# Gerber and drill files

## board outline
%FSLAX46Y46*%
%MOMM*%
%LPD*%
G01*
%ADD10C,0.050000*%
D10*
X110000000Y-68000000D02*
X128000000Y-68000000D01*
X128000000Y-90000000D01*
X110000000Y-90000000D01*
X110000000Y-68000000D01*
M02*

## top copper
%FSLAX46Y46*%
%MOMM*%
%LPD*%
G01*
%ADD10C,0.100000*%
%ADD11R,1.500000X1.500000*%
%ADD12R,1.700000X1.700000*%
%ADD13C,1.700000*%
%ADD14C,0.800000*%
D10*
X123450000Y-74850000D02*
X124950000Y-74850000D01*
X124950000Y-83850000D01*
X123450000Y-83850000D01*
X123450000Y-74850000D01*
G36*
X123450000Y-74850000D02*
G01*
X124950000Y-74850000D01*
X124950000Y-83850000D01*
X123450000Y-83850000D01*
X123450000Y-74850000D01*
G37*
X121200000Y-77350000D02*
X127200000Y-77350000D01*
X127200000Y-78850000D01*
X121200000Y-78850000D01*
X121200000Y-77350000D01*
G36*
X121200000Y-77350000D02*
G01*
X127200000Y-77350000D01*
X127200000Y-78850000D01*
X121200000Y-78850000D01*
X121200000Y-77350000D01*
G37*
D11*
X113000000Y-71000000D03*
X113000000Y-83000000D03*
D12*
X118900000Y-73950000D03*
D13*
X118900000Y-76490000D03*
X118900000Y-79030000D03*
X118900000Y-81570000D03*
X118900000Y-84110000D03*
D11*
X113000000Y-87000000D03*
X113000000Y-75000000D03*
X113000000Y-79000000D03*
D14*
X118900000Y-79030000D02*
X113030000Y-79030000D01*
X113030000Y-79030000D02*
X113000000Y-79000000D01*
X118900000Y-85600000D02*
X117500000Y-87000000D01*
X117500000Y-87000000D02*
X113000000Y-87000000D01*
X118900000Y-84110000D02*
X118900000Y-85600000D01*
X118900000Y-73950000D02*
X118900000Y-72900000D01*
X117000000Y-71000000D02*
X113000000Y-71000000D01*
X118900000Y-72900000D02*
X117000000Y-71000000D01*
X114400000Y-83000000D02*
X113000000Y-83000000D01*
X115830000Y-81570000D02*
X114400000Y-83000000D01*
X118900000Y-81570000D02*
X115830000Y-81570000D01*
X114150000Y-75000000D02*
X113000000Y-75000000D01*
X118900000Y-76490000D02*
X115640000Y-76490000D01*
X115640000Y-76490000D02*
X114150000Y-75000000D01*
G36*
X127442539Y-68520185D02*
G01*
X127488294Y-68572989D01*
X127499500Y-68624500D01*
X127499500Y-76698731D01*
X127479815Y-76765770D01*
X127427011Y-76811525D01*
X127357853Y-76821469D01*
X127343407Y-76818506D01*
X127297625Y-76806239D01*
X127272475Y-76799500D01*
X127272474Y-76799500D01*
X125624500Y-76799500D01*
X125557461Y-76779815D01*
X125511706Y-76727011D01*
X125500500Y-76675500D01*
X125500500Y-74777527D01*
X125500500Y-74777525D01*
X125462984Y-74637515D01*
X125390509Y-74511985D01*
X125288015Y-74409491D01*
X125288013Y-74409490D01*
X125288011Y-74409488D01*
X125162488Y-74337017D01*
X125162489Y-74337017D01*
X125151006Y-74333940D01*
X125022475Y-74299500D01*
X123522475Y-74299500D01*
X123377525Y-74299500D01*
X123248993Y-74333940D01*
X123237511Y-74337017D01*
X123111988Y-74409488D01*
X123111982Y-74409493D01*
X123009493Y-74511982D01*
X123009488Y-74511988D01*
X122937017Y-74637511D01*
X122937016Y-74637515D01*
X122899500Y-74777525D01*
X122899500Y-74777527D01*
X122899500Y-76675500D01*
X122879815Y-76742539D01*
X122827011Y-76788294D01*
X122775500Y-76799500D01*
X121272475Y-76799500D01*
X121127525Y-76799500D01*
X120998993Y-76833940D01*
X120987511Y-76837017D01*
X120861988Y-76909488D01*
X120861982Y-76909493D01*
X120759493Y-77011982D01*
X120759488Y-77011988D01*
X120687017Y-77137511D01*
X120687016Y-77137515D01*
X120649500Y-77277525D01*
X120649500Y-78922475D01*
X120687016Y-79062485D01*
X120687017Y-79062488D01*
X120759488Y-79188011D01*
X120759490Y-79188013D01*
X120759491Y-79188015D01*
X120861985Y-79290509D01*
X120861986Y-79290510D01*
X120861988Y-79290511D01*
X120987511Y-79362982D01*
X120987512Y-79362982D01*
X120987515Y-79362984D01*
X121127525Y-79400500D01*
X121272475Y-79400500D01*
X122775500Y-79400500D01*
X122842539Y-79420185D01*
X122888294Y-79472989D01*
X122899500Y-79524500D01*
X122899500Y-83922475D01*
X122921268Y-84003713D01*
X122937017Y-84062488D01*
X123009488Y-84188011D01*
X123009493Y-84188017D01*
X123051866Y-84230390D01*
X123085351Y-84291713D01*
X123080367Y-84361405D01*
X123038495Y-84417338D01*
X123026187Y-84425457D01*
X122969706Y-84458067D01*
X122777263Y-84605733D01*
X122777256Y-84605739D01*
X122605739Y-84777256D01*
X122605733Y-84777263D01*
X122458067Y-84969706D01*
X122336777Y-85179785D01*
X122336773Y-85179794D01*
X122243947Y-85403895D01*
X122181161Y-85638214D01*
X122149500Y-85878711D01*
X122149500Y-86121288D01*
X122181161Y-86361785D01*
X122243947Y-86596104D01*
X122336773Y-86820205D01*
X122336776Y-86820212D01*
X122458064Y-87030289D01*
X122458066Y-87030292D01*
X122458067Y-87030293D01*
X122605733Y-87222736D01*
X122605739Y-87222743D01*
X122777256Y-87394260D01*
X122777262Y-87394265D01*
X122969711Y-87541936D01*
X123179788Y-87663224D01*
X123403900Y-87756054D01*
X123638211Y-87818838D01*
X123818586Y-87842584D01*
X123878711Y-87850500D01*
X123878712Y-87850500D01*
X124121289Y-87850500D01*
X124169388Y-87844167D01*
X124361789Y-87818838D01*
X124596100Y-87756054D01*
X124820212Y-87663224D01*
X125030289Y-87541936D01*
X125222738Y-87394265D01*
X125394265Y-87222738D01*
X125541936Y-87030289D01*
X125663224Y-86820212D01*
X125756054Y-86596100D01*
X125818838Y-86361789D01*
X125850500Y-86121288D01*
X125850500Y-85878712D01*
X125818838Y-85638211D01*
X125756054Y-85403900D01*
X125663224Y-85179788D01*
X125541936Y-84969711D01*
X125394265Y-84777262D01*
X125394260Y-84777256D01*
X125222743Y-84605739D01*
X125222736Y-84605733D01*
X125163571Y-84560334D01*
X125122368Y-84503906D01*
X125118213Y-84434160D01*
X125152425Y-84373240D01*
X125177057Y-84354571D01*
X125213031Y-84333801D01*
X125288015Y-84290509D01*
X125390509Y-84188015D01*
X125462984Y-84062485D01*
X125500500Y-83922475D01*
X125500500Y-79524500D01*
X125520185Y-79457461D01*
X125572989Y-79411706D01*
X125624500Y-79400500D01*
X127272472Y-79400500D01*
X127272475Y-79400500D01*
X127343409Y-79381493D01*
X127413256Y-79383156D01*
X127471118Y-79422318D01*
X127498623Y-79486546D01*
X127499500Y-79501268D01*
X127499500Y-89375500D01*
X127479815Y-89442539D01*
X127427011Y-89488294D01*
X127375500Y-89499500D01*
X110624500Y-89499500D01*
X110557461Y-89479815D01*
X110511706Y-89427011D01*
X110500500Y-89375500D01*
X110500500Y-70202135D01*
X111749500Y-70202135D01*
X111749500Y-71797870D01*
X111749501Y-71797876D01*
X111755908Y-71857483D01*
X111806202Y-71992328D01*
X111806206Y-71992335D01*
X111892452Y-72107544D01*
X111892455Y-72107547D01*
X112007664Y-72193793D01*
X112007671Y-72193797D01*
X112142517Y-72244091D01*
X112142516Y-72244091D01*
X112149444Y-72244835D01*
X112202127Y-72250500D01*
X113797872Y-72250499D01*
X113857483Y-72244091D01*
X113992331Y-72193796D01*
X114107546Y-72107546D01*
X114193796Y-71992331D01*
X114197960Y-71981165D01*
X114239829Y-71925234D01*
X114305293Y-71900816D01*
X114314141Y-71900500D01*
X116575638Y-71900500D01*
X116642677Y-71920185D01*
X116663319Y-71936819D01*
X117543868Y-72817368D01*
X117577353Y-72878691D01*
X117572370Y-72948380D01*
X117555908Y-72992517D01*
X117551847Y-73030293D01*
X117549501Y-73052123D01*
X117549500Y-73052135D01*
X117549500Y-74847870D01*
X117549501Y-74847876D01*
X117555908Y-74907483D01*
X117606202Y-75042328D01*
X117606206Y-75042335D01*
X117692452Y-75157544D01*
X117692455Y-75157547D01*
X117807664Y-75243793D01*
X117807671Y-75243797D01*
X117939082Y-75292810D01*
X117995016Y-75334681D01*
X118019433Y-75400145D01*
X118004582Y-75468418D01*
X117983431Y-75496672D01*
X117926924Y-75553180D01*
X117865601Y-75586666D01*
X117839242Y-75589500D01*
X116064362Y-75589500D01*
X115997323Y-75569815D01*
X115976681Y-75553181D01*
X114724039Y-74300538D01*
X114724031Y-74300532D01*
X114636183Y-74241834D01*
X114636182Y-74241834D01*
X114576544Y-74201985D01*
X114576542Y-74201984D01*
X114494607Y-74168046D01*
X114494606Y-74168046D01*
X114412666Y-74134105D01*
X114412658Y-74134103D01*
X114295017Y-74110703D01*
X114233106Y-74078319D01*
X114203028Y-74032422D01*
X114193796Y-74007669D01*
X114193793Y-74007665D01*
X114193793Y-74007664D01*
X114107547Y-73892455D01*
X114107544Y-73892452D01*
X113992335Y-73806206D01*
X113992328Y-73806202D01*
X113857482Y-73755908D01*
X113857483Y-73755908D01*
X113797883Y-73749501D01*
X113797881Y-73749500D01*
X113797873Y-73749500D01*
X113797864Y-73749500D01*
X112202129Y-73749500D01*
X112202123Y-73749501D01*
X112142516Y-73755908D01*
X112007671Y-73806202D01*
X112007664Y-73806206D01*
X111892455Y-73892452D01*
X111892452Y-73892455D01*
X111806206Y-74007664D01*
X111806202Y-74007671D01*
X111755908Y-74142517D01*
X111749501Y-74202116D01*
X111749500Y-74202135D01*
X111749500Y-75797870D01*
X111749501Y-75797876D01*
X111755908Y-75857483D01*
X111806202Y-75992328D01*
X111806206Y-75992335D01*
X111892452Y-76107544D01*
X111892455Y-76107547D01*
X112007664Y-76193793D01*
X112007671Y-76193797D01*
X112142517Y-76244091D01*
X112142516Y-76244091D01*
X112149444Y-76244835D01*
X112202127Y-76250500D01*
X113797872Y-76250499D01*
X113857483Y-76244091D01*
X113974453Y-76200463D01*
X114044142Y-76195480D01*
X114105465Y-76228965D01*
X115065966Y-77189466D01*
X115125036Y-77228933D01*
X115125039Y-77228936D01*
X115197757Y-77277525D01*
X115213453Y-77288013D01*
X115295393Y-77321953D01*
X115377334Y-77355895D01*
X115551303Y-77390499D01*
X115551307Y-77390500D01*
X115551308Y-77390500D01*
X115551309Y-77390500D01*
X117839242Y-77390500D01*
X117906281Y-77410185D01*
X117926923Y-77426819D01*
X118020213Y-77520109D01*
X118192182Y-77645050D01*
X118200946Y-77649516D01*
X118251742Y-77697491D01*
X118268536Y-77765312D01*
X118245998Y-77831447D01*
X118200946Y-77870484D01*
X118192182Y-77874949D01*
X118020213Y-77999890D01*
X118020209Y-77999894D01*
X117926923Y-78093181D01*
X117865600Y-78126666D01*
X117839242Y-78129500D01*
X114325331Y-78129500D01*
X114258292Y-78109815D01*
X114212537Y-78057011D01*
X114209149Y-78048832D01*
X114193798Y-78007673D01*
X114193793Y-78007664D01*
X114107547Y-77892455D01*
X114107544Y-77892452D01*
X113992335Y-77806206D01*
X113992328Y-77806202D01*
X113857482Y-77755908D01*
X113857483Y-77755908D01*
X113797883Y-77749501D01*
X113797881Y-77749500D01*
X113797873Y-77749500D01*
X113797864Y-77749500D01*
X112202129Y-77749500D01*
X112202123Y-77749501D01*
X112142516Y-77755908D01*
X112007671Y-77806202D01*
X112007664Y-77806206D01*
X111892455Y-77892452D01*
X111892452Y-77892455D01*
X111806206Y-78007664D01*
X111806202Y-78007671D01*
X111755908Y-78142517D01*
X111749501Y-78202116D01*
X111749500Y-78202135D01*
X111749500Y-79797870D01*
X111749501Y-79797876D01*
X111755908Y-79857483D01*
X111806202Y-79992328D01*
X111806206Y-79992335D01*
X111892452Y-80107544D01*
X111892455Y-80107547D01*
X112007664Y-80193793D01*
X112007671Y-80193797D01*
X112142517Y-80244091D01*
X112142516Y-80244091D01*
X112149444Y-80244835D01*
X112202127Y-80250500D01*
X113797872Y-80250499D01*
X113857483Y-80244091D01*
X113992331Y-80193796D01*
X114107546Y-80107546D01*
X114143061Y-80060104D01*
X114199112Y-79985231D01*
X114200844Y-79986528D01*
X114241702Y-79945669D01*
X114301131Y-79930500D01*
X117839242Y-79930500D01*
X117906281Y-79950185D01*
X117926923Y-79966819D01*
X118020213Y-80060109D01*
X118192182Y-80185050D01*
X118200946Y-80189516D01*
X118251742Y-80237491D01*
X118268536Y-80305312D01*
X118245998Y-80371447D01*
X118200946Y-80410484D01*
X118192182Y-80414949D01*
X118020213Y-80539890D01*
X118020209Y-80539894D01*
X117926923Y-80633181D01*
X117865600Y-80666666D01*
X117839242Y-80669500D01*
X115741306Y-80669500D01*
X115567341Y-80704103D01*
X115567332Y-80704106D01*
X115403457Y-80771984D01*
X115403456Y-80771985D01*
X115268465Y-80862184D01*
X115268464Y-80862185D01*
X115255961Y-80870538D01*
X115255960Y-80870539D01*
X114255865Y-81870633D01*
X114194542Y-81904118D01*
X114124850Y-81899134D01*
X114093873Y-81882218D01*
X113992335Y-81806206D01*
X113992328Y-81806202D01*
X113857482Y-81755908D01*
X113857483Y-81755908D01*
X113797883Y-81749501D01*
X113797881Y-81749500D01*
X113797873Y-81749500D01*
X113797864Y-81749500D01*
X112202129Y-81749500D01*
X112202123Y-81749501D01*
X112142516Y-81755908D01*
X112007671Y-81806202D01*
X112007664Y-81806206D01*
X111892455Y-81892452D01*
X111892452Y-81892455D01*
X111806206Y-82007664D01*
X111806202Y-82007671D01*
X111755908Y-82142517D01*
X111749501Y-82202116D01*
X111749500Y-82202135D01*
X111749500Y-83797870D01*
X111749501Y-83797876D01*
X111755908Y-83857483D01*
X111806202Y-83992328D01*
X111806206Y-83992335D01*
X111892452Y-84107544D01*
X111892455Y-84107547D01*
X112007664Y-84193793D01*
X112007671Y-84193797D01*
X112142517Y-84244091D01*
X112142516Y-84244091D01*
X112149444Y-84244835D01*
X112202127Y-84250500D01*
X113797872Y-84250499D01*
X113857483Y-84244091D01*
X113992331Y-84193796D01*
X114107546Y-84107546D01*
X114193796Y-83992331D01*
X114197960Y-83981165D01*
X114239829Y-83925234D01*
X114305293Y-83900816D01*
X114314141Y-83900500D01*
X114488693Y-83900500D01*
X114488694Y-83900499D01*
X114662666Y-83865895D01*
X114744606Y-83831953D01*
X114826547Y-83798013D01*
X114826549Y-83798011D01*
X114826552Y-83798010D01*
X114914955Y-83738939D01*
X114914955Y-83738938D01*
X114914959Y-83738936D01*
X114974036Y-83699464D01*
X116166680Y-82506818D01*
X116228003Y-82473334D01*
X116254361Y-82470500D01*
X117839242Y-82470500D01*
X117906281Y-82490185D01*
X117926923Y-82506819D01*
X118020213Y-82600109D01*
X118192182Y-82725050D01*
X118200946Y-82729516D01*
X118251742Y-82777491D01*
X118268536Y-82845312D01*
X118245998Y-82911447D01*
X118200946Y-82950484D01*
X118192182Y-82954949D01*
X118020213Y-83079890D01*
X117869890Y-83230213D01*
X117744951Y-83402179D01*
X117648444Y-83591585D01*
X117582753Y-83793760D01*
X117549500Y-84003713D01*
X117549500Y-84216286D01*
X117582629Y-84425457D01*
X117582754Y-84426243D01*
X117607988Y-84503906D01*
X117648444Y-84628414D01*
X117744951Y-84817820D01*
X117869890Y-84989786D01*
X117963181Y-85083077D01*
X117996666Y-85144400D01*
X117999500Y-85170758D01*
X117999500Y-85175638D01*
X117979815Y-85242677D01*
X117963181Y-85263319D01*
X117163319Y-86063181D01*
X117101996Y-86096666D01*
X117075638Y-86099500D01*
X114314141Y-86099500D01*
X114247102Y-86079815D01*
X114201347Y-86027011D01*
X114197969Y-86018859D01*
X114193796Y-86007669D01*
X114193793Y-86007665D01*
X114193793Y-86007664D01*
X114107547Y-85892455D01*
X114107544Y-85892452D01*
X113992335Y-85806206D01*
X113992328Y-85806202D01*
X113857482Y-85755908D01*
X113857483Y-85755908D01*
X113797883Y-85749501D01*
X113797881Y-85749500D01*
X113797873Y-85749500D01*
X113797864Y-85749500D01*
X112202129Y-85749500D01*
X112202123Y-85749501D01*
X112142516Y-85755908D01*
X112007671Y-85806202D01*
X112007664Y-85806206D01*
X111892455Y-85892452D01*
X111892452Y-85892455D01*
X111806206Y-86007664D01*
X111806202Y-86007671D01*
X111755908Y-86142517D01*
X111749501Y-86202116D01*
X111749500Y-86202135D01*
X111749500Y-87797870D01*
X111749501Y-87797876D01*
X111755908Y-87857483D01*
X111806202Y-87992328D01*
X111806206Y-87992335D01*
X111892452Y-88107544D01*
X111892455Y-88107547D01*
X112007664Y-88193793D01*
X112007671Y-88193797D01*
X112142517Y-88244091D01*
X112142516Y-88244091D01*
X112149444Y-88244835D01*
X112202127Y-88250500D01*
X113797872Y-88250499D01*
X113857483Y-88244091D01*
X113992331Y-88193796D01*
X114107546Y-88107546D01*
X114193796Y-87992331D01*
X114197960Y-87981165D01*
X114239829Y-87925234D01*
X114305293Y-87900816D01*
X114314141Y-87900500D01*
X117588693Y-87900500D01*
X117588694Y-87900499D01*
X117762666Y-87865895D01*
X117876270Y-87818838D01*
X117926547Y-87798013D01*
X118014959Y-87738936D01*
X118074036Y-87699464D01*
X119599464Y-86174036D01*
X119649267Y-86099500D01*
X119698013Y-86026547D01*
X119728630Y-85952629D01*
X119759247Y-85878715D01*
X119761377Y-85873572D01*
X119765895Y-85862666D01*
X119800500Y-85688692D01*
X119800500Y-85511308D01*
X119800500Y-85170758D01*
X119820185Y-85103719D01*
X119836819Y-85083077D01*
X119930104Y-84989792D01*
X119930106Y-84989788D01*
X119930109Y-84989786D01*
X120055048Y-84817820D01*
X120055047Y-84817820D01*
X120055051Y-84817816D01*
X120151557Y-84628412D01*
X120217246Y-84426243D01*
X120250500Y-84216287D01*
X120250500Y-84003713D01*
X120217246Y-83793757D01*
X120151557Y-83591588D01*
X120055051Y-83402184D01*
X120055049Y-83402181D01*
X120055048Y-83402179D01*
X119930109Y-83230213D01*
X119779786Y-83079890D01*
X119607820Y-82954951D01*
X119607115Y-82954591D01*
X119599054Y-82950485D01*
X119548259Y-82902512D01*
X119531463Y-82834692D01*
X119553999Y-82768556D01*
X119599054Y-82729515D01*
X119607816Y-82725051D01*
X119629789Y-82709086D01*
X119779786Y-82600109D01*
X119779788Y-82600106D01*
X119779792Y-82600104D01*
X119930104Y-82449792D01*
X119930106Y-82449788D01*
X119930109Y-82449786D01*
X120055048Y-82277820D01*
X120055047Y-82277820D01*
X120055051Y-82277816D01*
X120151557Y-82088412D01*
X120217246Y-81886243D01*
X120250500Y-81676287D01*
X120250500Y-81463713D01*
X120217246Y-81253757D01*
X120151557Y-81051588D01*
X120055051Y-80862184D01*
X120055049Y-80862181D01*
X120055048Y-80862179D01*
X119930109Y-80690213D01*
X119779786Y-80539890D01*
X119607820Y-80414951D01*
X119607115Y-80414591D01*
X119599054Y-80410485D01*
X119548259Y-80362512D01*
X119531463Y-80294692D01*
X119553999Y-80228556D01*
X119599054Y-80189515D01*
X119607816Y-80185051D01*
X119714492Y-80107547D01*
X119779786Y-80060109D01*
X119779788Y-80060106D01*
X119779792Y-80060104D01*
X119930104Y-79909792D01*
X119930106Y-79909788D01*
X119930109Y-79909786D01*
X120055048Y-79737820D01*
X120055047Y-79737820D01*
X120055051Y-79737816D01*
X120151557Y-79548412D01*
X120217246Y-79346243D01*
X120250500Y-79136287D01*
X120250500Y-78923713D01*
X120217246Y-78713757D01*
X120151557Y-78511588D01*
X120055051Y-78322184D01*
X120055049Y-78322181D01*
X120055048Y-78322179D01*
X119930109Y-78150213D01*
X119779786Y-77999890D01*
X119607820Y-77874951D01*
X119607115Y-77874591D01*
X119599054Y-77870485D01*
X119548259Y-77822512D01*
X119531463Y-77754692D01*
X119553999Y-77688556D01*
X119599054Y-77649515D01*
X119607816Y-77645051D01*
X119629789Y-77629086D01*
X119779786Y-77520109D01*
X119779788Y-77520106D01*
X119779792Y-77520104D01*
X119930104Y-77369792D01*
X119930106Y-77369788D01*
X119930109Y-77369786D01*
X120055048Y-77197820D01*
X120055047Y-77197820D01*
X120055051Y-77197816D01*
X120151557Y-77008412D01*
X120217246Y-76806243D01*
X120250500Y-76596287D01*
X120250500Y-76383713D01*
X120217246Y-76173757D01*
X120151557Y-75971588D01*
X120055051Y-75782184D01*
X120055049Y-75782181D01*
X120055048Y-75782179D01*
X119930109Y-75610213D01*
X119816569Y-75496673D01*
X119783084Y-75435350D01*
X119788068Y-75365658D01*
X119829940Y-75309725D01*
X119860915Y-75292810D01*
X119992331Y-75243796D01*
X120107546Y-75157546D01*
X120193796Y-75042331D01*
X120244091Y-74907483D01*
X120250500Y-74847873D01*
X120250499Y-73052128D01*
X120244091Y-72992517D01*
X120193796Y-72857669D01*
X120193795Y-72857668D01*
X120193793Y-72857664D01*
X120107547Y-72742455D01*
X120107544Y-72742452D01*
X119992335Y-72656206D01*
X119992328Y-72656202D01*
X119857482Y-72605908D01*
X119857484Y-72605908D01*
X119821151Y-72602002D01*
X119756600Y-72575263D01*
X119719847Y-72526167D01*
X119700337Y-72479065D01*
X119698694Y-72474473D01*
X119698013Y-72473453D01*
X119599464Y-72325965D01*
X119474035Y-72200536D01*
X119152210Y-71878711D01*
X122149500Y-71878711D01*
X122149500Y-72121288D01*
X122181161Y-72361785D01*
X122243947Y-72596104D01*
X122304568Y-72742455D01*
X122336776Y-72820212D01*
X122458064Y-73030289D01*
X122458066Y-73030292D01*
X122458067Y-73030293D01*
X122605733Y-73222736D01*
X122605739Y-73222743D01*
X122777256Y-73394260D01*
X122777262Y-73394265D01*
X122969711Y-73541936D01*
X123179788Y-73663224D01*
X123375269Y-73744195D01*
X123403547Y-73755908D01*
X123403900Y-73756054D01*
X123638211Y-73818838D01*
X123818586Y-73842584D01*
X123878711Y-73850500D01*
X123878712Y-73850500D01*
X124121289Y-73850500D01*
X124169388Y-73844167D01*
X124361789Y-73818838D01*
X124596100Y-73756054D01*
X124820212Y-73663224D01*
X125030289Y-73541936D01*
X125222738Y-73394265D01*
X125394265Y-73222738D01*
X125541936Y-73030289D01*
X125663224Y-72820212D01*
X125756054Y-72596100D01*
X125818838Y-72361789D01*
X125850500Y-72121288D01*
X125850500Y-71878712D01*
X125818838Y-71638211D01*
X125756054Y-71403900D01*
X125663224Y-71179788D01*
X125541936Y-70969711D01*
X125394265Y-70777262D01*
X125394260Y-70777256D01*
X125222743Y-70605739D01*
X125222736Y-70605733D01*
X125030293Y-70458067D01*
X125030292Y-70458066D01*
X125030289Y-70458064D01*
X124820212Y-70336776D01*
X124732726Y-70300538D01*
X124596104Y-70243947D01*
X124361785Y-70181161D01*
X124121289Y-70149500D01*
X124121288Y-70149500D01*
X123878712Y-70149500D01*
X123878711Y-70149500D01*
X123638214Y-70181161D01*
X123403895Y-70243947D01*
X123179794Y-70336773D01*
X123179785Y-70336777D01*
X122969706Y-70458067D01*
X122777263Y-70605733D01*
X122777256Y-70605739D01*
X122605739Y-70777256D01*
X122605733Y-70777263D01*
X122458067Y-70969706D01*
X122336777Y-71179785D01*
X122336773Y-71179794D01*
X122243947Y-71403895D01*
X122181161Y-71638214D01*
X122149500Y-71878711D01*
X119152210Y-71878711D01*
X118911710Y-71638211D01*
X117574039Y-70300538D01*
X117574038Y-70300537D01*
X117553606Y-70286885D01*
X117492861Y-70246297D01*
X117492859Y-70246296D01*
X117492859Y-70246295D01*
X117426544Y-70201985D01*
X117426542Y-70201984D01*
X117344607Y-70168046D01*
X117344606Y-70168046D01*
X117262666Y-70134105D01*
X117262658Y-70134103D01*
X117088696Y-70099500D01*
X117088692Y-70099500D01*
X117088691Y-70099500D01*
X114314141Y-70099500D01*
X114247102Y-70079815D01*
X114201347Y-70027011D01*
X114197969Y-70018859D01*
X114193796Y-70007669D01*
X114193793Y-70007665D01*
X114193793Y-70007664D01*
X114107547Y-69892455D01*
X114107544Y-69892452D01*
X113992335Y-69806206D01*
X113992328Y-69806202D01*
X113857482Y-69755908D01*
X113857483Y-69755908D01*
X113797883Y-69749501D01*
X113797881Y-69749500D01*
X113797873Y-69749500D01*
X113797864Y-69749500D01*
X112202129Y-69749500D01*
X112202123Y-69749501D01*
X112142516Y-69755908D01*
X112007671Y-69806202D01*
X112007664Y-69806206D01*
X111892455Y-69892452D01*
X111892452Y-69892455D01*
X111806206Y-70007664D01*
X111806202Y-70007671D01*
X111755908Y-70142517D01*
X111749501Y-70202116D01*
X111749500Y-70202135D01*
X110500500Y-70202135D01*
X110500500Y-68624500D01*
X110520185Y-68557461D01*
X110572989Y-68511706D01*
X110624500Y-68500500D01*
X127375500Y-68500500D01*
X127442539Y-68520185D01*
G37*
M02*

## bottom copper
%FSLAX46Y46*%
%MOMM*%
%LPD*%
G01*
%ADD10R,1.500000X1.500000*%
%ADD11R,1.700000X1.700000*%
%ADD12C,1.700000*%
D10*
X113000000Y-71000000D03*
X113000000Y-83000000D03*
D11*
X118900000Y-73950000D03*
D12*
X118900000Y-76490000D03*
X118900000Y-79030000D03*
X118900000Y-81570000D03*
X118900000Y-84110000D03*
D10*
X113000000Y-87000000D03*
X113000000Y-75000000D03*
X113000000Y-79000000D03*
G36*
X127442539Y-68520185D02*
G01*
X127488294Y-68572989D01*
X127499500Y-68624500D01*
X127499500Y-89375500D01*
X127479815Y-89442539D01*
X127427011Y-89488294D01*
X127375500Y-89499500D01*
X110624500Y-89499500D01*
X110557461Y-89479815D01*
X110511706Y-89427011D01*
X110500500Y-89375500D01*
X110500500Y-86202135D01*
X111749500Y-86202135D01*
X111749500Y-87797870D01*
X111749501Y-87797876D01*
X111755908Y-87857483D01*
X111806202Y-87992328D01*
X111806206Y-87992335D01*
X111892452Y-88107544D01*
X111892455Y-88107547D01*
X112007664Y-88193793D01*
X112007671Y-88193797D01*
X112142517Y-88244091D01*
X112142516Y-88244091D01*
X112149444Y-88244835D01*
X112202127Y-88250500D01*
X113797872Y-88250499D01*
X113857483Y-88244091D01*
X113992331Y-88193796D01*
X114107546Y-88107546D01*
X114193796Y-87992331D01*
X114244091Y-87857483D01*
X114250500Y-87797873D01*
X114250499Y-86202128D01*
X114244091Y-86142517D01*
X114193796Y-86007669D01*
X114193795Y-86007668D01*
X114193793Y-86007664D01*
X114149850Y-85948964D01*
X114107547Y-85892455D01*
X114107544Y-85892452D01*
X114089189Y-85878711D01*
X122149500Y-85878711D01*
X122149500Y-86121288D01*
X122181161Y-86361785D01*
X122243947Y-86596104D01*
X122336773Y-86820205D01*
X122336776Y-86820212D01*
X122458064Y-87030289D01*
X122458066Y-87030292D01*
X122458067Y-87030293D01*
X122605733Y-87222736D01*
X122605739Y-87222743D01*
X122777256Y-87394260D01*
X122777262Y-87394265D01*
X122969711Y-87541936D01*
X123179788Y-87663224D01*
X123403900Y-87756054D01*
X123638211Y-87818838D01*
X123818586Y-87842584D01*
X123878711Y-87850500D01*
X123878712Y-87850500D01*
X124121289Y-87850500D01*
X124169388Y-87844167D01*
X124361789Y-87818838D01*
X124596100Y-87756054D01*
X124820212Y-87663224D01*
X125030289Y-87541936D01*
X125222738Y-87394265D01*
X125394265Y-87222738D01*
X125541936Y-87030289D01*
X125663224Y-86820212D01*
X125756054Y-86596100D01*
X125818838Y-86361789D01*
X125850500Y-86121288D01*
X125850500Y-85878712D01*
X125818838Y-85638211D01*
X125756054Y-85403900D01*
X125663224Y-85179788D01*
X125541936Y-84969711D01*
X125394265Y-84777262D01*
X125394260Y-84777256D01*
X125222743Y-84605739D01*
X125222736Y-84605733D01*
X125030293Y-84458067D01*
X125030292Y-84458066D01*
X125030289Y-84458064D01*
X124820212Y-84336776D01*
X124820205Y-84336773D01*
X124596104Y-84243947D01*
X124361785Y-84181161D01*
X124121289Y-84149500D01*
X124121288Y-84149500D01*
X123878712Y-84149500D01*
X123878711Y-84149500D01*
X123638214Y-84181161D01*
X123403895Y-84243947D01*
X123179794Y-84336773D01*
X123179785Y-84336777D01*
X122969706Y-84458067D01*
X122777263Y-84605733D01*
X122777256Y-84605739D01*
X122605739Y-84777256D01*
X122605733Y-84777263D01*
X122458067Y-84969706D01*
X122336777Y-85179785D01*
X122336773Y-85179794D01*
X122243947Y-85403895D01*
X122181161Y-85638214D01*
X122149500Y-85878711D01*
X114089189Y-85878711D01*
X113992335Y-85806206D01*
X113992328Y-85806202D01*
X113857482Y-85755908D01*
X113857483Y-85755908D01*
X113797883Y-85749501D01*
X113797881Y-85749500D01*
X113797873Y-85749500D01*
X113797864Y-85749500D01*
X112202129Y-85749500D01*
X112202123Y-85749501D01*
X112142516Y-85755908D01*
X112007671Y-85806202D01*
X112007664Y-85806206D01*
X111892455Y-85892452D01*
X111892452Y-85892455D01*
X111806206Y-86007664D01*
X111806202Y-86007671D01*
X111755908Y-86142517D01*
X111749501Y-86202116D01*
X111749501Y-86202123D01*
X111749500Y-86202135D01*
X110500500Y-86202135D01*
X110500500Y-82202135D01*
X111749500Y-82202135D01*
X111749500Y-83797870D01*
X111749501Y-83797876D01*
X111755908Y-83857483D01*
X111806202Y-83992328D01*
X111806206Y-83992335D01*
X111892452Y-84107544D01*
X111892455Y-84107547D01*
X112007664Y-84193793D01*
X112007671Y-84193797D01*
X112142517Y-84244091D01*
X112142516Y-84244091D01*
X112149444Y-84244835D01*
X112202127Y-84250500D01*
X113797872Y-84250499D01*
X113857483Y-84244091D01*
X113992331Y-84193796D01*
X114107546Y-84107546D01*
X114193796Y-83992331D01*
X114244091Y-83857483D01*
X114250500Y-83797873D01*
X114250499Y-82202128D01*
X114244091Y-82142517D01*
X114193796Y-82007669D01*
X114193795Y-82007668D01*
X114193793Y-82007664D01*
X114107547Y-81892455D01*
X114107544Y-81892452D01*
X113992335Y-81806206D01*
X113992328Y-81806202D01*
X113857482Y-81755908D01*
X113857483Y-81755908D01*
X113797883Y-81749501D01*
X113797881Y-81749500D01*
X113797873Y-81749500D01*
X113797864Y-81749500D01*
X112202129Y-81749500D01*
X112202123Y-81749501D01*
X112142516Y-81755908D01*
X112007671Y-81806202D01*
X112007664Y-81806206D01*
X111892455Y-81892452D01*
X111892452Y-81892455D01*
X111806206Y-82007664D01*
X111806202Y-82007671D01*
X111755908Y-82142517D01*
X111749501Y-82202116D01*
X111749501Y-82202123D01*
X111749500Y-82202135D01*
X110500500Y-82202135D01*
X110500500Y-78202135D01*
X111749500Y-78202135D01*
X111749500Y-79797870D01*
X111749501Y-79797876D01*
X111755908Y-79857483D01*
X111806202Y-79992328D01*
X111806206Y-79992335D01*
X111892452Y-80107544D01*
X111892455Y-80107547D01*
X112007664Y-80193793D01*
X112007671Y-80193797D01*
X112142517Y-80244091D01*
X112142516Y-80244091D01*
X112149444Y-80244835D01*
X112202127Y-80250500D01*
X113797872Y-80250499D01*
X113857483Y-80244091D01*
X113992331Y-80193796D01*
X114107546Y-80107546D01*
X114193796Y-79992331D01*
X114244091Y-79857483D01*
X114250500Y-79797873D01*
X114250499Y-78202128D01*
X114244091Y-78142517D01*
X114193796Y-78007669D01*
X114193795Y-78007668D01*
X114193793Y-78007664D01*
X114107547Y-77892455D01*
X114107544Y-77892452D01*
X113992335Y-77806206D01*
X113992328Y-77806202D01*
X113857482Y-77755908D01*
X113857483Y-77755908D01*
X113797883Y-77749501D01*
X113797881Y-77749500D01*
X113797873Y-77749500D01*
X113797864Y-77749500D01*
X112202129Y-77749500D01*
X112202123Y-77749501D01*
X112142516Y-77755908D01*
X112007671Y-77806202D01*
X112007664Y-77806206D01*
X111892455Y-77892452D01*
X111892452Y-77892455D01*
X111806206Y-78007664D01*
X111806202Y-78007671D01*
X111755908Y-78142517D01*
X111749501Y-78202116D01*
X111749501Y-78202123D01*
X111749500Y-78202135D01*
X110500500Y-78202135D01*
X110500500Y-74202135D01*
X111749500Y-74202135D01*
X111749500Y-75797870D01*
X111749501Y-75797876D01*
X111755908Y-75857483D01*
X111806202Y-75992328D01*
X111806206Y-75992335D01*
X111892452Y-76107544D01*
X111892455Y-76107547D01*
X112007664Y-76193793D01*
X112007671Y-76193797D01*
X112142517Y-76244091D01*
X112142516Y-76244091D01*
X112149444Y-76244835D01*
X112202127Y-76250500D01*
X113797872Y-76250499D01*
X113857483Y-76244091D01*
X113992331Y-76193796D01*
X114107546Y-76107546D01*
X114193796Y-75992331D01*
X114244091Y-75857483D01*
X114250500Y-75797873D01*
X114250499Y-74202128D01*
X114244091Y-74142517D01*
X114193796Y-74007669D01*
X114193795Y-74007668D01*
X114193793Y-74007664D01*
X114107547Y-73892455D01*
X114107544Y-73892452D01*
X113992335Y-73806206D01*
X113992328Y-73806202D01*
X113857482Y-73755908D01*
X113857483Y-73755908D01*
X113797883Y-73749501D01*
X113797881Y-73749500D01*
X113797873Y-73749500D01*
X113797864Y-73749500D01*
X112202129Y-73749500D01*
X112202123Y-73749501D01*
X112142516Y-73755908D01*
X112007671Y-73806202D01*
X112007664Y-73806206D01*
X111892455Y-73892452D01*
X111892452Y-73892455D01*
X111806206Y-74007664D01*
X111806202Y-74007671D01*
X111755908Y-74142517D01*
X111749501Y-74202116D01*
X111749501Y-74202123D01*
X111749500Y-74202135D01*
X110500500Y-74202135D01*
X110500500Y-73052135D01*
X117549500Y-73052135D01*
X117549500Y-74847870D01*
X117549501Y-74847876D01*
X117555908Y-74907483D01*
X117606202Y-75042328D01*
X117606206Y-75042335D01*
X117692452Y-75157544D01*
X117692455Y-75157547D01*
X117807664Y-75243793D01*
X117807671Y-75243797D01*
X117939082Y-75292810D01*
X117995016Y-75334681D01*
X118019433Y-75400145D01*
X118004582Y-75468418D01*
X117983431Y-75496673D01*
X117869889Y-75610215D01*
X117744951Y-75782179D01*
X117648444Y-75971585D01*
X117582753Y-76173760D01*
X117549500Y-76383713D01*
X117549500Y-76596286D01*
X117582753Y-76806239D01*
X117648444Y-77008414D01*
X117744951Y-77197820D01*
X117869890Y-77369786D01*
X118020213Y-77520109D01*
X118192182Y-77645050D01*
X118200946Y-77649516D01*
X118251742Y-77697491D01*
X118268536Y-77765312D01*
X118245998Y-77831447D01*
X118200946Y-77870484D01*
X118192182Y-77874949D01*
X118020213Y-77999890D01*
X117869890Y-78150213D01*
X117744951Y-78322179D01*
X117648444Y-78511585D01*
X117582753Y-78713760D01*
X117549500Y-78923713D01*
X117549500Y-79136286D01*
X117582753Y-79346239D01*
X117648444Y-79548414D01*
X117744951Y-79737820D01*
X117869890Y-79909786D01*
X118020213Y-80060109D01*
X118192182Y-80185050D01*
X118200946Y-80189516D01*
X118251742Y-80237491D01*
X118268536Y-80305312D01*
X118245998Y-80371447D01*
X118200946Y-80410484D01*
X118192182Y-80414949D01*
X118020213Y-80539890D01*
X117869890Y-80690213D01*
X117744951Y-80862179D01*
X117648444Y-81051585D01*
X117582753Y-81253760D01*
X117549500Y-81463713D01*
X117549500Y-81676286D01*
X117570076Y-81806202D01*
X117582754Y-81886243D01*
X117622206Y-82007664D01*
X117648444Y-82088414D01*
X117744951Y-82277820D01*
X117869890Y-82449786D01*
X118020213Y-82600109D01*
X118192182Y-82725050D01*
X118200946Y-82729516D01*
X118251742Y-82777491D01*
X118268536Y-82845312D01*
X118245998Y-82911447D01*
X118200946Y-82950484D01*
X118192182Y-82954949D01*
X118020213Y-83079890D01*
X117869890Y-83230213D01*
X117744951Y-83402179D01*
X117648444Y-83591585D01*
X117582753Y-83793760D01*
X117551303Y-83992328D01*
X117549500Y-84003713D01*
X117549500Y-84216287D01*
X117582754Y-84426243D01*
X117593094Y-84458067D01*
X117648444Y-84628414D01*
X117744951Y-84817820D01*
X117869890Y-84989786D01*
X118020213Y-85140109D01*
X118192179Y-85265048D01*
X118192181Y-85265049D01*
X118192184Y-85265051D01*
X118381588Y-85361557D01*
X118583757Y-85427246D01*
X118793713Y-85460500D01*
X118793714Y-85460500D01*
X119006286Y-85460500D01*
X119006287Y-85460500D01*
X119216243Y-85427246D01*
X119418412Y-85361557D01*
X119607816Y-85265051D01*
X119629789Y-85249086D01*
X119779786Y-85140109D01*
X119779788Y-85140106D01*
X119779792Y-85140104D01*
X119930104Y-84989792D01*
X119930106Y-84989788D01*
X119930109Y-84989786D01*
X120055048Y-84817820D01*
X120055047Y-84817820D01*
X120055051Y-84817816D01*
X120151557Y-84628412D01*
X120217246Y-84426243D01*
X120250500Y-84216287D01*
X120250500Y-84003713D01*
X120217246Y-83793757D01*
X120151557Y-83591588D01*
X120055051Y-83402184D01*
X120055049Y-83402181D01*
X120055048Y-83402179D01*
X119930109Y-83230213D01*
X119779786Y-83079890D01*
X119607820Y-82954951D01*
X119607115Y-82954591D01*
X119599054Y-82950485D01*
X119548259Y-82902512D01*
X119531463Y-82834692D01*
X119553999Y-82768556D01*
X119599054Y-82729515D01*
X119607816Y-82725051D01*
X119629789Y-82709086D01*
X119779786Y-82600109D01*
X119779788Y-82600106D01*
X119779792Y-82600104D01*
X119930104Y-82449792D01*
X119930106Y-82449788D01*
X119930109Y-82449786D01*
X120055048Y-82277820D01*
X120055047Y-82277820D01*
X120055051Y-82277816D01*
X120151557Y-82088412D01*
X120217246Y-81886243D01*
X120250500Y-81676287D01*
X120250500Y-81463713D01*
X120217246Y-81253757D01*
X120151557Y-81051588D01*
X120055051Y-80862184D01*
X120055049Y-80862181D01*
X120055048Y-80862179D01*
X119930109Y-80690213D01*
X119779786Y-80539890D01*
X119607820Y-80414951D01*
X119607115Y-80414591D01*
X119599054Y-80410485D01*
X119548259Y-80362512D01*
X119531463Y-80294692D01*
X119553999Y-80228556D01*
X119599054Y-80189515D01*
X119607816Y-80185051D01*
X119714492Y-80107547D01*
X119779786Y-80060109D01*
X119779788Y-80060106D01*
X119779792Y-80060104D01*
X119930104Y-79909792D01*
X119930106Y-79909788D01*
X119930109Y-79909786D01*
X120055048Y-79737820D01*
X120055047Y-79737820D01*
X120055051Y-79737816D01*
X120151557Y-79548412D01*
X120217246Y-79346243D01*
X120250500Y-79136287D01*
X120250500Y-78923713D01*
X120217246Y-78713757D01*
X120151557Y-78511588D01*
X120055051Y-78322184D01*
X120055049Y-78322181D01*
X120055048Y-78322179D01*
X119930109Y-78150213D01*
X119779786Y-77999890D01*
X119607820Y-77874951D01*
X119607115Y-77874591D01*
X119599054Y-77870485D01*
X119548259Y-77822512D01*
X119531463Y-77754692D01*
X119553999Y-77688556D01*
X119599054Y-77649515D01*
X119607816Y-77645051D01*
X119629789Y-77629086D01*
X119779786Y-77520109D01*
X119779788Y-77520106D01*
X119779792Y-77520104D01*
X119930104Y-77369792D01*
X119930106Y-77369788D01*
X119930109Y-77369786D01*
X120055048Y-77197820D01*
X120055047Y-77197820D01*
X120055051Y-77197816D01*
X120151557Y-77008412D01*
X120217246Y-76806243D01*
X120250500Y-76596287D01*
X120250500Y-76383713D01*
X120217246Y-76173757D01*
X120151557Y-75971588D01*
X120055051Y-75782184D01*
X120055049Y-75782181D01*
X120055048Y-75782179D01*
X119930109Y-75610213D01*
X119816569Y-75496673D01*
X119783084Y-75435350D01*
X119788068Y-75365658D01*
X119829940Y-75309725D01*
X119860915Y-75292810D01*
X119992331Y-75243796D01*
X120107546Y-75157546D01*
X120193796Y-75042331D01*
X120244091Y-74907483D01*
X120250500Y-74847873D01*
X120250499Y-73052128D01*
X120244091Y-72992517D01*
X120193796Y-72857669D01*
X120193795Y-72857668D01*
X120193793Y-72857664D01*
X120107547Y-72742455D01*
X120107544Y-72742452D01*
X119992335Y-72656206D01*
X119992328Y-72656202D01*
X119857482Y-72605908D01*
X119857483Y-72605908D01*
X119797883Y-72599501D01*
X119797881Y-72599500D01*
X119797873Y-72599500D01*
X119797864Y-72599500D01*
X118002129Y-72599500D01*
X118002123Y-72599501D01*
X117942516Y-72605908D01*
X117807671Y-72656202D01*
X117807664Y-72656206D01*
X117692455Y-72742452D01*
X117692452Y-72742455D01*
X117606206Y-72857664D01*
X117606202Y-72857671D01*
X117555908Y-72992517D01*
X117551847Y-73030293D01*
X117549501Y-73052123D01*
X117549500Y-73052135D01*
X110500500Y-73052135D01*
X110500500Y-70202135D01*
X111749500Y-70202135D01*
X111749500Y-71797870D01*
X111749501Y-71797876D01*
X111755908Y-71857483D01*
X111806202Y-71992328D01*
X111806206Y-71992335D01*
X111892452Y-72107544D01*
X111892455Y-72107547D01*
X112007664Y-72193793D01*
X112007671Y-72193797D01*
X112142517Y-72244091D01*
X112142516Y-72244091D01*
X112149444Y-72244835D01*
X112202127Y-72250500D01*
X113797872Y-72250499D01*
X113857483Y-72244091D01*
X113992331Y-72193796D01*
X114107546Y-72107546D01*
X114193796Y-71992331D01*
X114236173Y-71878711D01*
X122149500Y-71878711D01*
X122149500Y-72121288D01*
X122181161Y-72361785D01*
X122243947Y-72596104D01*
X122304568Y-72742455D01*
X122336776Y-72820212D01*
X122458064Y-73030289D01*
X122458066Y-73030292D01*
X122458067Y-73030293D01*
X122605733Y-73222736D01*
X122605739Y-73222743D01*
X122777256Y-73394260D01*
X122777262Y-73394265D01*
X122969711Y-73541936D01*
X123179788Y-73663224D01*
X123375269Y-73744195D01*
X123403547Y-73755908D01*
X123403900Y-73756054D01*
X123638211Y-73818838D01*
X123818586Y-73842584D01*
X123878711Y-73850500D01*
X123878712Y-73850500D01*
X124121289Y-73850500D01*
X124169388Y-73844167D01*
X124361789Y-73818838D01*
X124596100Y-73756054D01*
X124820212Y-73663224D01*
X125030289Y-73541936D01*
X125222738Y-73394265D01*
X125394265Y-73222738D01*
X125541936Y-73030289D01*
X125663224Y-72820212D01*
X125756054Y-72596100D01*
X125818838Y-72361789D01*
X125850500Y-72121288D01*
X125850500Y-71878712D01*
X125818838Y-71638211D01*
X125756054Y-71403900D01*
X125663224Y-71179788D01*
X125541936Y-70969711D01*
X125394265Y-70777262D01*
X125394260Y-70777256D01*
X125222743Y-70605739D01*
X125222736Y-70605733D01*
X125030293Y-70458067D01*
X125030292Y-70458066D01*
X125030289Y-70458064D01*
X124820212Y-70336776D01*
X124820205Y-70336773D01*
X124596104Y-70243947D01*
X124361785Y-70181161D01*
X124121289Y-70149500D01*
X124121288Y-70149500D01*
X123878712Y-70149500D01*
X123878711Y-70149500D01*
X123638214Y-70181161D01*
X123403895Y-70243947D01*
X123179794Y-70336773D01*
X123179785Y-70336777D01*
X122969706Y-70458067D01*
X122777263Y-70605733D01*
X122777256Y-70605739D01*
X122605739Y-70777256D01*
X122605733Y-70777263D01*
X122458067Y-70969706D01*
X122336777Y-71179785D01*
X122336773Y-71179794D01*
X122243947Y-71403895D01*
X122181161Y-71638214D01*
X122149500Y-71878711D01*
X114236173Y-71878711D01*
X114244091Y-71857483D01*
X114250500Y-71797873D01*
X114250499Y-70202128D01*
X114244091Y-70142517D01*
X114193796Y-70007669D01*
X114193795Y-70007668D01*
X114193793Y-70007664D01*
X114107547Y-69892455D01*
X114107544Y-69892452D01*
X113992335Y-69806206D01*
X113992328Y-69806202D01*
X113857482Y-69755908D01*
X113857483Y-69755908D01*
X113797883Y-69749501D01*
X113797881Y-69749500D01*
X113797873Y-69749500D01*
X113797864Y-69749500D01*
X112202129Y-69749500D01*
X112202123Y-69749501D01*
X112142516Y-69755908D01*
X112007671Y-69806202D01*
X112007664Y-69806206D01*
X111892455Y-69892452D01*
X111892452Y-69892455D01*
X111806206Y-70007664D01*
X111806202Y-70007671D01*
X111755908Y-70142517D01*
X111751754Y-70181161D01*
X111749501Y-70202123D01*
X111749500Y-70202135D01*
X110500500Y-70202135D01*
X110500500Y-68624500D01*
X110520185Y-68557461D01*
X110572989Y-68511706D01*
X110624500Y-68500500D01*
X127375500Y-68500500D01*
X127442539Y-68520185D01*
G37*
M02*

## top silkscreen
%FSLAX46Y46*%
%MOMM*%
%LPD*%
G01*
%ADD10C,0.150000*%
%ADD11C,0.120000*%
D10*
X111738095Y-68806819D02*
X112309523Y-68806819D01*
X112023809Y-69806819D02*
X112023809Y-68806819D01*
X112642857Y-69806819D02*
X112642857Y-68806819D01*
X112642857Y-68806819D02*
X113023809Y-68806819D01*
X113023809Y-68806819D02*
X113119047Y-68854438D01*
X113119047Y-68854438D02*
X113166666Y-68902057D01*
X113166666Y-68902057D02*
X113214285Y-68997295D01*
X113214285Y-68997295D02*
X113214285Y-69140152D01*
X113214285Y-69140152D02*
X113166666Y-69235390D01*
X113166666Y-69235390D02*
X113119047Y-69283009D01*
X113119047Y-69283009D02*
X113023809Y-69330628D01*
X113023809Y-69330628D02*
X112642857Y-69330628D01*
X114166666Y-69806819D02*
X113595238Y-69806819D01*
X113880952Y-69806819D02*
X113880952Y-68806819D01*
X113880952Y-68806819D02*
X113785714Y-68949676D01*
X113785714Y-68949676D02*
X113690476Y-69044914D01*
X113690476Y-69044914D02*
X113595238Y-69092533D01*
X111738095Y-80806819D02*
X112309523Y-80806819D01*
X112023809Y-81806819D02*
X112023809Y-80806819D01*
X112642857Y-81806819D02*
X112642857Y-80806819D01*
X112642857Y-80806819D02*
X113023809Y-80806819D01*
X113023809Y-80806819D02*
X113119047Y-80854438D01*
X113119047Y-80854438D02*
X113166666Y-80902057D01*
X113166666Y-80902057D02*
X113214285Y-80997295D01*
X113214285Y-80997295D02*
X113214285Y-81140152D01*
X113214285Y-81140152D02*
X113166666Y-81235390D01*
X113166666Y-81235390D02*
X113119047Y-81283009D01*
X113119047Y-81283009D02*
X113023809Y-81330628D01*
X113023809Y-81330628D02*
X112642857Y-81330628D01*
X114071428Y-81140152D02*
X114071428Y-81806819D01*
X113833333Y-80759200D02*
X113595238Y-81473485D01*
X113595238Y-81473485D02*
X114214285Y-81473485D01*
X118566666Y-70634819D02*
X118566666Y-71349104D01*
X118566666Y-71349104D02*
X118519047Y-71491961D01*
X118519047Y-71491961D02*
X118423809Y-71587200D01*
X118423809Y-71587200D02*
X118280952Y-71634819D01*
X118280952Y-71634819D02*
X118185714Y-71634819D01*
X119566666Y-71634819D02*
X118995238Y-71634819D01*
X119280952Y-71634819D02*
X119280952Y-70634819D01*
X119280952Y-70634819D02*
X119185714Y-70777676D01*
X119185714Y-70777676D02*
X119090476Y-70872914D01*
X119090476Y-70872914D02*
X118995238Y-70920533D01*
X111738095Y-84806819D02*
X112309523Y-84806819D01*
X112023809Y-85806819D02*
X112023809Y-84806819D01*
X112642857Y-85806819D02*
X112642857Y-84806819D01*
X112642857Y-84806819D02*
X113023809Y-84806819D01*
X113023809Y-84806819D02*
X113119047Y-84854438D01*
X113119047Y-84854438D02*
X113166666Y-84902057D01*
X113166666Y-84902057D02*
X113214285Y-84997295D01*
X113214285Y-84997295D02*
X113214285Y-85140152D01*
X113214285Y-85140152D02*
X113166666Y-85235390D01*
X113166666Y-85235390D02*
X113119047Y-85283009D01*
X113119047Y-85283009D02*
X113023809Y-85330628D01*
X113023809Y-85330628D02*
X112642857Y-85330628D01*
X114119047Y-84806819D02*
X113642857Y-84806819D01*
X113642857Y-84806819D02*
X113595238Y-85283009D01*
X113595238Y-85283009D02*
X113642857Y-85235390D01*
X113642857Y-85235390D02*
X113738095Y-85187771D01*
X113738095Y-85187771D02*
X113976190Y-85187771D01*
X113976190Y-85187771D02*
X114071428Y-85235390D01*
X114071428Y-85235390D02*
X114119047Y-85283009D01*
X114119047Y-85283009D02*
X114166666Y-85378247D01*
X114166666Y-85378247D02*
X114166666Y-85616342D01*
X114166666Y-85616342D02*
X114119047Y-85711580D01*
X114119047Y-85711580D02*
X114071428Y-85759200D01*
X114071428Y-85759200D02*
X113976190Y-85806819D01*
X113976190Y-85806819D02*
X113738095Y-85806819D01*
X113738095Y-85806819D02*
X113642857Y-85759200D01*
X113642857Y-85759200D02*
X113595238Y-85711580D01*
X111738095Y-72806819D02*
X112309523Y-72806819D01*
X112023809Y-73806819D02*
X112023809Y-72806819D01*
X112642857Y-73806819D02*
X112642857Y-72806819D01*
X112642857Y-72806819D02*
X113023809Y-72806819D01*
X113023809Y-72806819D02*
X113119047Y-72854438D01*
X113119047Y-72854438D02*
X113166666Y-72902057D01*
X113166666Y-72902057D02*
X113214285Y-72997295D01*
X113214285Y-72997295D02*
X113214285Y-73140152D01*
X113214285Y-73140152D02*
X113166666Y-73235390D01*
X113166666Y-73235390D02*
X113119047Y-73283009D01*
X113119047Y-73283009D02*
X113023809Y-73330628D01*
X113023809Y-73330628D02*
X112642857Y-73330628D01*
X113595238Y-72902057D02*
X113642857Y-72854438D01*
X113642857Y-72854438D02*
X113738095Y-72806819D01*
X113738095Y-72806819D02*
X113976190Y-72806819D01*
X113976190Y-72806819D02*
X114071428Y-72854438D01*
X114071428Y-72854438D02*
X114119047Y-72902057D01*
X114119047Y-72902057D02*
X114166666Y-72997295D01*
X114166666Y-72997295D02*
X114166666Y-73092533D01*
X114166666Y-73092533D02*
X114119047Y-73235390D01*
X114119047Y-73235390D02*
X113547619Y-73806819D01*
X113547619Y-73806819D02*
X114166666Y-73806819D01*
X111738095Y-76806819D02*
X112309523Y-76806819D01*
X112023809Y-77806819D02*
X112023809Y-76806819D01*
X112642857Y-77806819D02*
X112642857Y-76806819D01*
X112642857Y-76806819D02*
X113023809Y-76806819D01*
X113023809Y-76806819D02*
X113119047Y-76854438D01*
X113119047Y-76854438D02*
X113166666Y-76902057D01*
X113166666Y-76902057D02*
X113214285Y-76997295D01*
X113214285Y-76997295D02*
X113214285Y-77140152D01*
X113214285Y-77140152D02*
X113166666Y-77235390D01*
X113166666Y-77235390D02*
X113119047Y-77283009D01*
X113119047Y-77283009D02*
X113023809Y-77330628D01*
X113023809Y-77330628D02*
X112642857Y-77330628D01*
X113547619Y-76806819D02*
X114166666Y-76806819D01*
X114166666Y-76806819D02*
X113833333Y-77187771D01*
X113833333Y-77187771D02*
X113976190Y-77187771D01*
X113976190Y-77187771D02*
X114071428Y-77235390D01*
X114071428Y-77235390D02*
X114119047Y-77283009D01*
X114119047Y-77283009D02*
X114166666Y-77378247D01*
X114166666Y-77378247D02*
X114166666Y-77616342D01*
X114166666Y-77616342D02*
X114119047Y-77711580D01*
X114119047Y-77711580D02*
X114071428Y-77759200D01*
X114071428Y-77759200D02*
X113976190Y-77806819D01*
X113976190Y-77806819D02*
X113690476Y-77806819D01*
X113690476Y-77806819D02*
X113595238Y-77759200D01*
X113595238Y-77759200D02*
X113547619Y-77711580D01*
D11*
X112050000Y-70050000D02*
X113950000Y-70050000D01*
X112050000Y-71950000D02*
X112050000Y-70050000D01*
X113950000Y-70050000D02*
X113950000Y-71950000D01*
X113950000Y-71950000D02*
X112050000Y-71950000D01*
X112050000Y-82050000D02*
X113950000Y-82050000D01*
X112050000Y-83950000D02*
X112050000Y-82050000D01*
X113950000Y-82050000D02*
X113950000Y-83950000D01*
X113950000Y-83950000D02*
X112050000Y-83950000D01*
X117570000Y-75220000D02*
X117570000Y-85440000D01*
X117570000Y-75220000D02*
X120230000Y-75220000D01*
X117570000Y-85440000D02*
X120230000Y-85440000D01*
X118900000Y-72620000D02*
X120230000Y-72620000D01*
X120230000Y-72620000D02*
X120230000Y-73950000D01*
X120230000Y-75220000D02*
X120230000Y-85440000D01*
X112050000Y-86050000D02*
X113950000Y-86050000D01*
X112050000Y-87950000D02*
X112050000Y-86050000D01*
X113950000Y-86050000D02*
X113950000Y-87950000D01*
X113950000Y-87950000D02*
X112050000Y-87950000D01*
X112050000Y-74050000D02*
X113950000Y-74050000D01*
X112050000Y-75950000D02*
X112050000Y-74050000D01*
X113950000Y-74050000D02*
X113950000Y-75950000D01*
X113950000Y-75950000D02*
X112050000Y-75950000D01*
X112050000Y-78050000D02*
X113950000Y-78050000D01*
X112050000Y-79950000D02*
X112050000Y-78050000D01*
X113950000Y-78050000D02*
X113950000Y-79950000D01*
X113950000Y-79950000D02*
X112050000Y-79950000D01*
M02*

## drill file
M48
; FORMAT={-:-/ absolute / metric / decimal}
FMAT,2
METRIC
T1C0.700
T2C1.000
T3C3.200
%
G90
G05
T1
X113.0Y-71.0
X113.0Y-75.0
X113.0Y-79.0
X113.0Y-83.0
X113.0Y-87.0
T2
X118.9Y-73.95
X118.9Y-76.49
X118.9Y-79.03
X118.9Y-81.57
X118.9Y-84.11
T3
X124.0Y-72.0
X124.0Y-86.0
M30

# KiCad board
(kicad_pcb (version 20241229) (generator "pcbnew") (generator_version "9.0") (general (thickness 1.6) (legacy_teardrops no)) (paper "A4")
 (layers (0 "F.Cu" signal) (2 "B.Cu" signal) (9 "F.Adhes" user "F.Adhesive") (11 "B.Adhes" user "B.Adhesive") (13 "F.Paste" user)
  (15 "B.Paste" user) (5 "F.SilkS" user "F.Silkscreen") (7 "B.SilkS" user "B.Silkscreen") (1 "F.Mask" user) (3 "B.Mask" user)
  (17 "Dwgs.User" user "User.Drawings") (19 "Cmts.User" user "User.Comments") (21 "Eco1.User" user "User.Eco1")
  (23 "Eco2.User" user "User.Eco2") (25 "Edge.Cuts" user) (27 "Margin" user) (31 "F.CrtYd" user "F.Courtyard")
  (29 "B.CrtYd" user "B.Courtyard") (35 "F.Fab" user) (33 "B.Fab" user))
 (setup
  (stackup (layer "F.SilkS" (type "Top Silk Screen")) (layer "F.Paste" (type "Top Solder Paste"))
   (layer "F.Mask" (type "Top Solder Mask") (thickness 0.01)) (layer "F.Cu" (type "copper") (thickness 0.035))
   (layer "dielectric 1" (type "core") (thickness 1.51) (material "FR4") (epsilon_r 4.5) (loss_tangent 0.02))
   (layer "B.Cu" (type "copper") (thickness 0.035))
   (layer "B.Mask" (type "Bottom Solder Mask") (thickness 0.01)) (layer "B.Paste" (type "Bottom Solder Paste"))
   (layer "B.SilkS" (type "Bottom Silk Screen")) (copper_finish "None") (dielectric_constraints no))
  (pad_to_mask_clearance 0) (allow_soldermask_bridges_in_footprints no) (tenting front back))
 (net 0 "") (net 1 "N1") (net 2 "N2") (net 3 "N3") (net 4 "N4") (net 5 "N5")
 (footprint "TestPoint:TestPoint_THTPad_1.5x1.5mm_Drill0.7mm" (layer "F.Cu") (at 113 71)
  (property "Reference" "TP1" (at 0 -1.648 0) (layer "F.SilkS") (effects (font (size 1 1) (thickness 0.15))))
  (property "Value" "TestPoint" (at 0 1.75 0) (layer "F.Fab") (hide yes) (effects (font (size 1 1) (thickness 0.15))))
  (fp_line (start -0.95 -0.95) (end 0.95 -0.95) (stroke (width 0.12) (type solid)) (layer "F.SilkS"))
  (fp_line (start -0.95 0.95) (end -0.95 -0.95) (stroke (width 0.12) (type solid)) (layer "F.SilkS"))
  (fp_line (start 0.95 -0.95) (end 0.95 0.95) (stroke (width 0.12) (type solid)) (layer "F.SilkS"))
  (fp_line (start 0.95 0.95) (end -0.95 0.95) (stroke (width 0.12) (type solid)) (layer "F.SilkS"))
  (pad "1" thru_hole rect (at 0 0) (size 1.5 1.5) (drill 0.7) (layers "*.Cu" "*.Mask") (remove_unused_layers no) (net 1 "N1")))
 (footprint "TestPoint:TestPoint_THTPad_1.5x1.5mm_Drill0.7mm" (layer "F.Cu") (at 113 83)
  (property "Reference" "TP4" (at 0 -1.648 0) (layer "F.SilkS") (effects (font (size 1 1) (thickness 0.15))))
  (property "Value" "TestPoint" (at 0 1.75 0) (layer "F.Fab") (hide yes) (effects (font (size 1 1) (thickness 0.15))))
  (fp_line (start -0.95 -0.95) (end 0.95 -0.95) (stroke (width 0.12) (type solid)) (layer "F.SilkS"))
  (fp_line (start -0.95 0.95) (end -0.95 -0.95) (stroke (width 0.12) (type solid)) (layer "F.SilkS"))
  (fp_line (start 0.95 -0.95) (end 0.95 0.95) (stroke (width 0.12) (type solid)) (layer "F.SilkS"))
  (fp_line (start 0.95 0.95) (end -0.95 0.95) (stroke (width 0.12) (type solid)) (layer "F.SilkS"))
  (pad "1" thru_hole rect (at 0 0) (size 1.5 1.5) (drill 0.7) (layers "*.Cu" "*.Mask") (remove_unused_layers no) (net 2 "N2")))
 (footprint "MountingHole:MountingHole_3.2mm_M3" (layer "F.Cu") (at 124 72)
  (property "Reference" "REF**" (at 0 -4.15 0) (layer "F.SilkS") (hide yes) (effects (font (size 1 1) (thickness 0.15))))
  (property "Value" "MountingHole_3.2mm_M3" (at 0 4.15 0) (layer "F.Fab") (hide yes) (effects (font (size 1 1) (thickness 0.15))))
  (pad "" np_thru_hole circle (at 0 0) (size 3.2 3.2) (drill 3.2) (layers "*.Cu" "*.Mask")))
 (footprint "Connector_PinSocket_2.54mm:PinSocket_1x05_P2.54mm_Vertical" (layer "F.Cu") (at 118.9 73.95)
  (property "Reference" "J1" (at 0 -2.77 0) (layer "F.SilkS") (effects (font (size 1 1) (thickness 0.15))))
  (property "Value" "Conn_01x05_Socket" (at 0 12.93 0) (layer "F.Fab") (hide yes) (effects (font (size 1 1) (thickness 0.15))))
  (fp_line (start -1.33 1.27) (end -1.33 11.49) (stroke (width 0.12) (type solid)) (layer "F.SilkS"))
  (fp_line (start -1.33 1.27) (end 1.33 1.27) (stroke (width 0.12) (type solid)) (layer "F.SilkS"))
  (fp_line (start -1.33 11.49) (end 1.33 11.49) (stroke (width 0.12) (type solid)) (layer "F.SilkS"))
  (fp_line (start 0 -1.33) (end 1.33 -1.33) (stroke (width 0.12) (type solid)) (layer "F.SilkS"))
  (fp_line (start 1.33 -1.33) (end 1.33 0) (stroke (width 0.12) (type solid)) (layer "F.SilkS"))
  (fp_line (start 1.33 1.27) (end 1.33 11.49) (stroke (width 0.12) (type solid)) (layer "F.SilkS"))
  (pad "1" thru_hole rect (at 0 0) (size 1.7 1.7) (drill 1) (layers "*.Cu" "*.Mask") (remove_unused_layers no) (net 1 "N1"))
  (pad "2" thru_hole circle (at 0 2.54) (size 1.7 1.7) (drill 1) (layers "*.Cu" "*.Mask") (remove_unused_layers no) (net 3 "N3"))
  (pad "3" thru_hole circle (at 0 5.08) (size 1.7 1.7) (drill 1) (layers "*.Cu" "*.Mask") (remove_unused_layers no) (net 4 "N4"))
  (pad "4" thru_hole circle (at 0 7.62) (size 1.7 1.7) (drill 1) (layers "*.Cu" "*.Mask") (remove_unused_layers no) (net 2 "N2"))
  (pad "5" thru_hole circle (at 0 10.16) (size 1.7 1.7) (drill 1) (layers "*.Cu" "*.Mask") (remove_unused_layers no) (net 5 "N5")))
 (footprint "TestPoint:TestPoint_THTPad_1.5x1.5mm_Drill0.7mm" (layer "F.Cu") (at 113 87)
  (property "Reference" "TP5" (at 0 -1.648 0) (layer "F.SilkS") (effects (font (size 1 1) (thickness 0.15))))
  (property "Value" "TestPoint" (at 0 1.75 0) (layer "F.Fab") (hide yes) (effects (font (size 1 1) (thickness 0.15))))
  (fp_line (start -0.95 -0.95) (end 0.95 -0.95) (stroke (width 0.12) (type solid)) (layer "F.SilkS"))
  (fp_line (start -0.95 0.95) (end -0.95 -0.95) (stroke (width 0.12) (type solid)) (layer "F.SilkS"))
  (fp_line (start 0.95 -0.95) (end 0.95 0.95) (stroke (width 0.12) (type solid)) (layer "F.SilkS"))
  (fp_line (start 0.95 0.95) (end -0.95 0.95) (stroke (width 0.12) (type solid)) (layer "F.SilkS"))
  (pad "1" thru_hole rect (at 0 0) (size 1.5 1.5) (drill 0.7) (layers "*.Cu" "*.Mask") (remove_unused_layers no) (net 5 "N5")))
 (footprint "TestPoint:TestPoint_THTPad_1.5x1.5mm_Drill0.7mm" (layer "F.Cu") (at 113 75)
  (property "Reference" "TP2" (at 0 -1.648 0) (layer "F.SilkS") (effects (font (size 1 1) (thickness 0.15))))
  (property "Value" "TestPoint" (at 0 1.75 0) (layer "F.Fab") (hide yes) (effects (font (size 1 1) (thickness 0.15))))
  (fp_line (start -0.95 -0.95) (end 0.95 -0.95) (stroke (width 0.12) (type solid)) (layer "F.SilkS"))
  (fp_line (start -0.95 0.95) (end -0.95 -0.95) (stroke (width 0.12) (type solid)) (layer "F.SilkS"))
  (fp_line (start 0.95 -0.95) (end 0.95 0.95) (stroke (width 0.12) (type solid)) (layer "F.SilkS"))
  (fp_line (start 0.95 0.95) (end -0.95 0.95) (stroke (width 0.12) (type solid)) (layer "F.SilkS"))
  (pad "1" thru_hole rect (at 0 0) (size 1.5 1.5) (drill 0.7) (layers "*.Cu" "*.Mask") (remove_unused_layers no) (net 3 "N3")))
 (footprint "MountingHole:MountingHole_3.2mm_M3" (layer "F.Cu") (at 124 86)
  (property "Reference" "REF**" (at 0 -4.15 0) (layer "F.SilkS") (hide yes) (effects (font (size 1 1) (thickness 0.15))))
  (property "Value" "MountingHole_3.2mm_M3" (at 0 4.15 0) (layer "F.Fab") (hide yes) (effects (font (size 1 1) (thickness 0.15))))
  (pad "" np_thru_hole circle (at 0 0) (size 3.2 3.2) (drill 3.2) (layers "*.Cu" "*.Mask")))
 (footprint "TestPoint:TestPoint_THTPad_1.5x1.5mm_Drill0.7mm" (layer "F.Cu") (at 113 79)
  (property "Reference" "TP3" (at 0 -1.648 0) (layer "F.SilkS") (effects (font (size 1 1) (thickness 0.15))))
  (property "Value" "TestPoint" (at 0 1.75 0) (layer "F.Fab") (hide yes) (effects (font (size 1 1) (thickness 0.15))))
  (fp_line (start -0.95 -0.95) (end 0.95 -0.95) (stroke (width 0.12) (type solid)) (layer "F.SilkS"))
  (fp_line (start -0.95 0.95) (end -0.95 -0.95) (stroke (width 0.12) (type solid)) (layer "F.SilkS"))
  (fp_line (start 0.95 -0.95) (end 0.95 0.95) (stroke (width 0.12) (type solid)) (layer "F.SilkS"))
  (fp_line (start 0.95 0.95) (end -0.95 0.95) (stroke (width 0.12) (type solid)) (layer "F.SilkS"))
  (pad "1" thru_hole rect (at 0 0) (size 1.5 1.5) (drill 0.7) (layers "*.Cu" "*.Mask") (remove_unused_layers no) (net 4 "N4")))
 (gr_rect (start 123.45 74.85) (end 124.95 83.85) (stroke (width 0.1) (type solid)) (fill yes) (layer "F.Cu"))
 (gr_rect (start 121.2 77.35) (end 127.2 78.85) (stroke (width 0.1) (type solid)) (fill yes) (layer "F.Cu"))
 (gr_rect (start 110 68) (end 128 90) (stroke (width 0.05) (type default)) (fill no) (layer "Edge.Cuts"))
 (segment (start 118.9 79.03) (end 113.03 79.03) (width 0.8) (layer "F.Cu") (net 4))
 (segment (start 113.03 79.03) (end 113 79) (width 0.8) (layer "F.Cu") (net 4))
 (segment (start 118.9 85.6) (end 117.5 87) (width 0.8) (layer "F.Cu") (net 5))
 (segment (start 117.5 87) (end 113 87) (width 0.8) (layer "F.Cu") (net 5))
 (segment (start 118.9 84.11) (end 118.9 85.6) (width 0.8) (layer "F.Cu") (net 5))
 (segment (start 118.9 73.95) (end 118.9 72.9) (width 0.8) (layer "F.Cu") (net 1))
 (segment (start 117 71) (end 113 71) (width 0.8) (layer "F.Cu") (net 1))
 (segment (start 118.9 72.9) (end 117 71) (width 0.8) (layer "F.Cu") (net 1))
 (segment (start 114.4 83) (end 113 83) (width 0.8) (layer "F.Cu") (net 2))
 (segment (start 115.83 81.57) (end 114.4 83) (width 0.8) (layer "F.Cu") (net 2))
 (segment (start 118.9 81.57) (end 115.83 81.57) (width 0.8) (layer "F.Cu") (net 2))
 (segment (start 114.15 75) (end 113 75) (width 0.8) (layer "F.Cu") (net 3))
 (segment (start 118.9 76.49) (end 115.64 76.49) (width 0.8) (layer "F.Cu") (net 3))
 (segment (start 115.64 76.49) (end 114.15 75) (width 0.8) (layer "F.Cu") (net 3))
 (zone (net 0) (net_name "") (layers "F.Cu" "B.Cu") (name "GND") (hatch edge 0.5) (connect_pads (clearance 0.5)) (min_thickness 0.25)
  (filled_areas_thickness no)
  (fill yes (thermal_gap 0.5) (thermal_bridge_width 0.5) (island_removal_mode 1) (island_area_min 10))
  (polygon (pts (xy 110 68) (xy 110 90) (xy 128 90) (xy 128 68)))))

